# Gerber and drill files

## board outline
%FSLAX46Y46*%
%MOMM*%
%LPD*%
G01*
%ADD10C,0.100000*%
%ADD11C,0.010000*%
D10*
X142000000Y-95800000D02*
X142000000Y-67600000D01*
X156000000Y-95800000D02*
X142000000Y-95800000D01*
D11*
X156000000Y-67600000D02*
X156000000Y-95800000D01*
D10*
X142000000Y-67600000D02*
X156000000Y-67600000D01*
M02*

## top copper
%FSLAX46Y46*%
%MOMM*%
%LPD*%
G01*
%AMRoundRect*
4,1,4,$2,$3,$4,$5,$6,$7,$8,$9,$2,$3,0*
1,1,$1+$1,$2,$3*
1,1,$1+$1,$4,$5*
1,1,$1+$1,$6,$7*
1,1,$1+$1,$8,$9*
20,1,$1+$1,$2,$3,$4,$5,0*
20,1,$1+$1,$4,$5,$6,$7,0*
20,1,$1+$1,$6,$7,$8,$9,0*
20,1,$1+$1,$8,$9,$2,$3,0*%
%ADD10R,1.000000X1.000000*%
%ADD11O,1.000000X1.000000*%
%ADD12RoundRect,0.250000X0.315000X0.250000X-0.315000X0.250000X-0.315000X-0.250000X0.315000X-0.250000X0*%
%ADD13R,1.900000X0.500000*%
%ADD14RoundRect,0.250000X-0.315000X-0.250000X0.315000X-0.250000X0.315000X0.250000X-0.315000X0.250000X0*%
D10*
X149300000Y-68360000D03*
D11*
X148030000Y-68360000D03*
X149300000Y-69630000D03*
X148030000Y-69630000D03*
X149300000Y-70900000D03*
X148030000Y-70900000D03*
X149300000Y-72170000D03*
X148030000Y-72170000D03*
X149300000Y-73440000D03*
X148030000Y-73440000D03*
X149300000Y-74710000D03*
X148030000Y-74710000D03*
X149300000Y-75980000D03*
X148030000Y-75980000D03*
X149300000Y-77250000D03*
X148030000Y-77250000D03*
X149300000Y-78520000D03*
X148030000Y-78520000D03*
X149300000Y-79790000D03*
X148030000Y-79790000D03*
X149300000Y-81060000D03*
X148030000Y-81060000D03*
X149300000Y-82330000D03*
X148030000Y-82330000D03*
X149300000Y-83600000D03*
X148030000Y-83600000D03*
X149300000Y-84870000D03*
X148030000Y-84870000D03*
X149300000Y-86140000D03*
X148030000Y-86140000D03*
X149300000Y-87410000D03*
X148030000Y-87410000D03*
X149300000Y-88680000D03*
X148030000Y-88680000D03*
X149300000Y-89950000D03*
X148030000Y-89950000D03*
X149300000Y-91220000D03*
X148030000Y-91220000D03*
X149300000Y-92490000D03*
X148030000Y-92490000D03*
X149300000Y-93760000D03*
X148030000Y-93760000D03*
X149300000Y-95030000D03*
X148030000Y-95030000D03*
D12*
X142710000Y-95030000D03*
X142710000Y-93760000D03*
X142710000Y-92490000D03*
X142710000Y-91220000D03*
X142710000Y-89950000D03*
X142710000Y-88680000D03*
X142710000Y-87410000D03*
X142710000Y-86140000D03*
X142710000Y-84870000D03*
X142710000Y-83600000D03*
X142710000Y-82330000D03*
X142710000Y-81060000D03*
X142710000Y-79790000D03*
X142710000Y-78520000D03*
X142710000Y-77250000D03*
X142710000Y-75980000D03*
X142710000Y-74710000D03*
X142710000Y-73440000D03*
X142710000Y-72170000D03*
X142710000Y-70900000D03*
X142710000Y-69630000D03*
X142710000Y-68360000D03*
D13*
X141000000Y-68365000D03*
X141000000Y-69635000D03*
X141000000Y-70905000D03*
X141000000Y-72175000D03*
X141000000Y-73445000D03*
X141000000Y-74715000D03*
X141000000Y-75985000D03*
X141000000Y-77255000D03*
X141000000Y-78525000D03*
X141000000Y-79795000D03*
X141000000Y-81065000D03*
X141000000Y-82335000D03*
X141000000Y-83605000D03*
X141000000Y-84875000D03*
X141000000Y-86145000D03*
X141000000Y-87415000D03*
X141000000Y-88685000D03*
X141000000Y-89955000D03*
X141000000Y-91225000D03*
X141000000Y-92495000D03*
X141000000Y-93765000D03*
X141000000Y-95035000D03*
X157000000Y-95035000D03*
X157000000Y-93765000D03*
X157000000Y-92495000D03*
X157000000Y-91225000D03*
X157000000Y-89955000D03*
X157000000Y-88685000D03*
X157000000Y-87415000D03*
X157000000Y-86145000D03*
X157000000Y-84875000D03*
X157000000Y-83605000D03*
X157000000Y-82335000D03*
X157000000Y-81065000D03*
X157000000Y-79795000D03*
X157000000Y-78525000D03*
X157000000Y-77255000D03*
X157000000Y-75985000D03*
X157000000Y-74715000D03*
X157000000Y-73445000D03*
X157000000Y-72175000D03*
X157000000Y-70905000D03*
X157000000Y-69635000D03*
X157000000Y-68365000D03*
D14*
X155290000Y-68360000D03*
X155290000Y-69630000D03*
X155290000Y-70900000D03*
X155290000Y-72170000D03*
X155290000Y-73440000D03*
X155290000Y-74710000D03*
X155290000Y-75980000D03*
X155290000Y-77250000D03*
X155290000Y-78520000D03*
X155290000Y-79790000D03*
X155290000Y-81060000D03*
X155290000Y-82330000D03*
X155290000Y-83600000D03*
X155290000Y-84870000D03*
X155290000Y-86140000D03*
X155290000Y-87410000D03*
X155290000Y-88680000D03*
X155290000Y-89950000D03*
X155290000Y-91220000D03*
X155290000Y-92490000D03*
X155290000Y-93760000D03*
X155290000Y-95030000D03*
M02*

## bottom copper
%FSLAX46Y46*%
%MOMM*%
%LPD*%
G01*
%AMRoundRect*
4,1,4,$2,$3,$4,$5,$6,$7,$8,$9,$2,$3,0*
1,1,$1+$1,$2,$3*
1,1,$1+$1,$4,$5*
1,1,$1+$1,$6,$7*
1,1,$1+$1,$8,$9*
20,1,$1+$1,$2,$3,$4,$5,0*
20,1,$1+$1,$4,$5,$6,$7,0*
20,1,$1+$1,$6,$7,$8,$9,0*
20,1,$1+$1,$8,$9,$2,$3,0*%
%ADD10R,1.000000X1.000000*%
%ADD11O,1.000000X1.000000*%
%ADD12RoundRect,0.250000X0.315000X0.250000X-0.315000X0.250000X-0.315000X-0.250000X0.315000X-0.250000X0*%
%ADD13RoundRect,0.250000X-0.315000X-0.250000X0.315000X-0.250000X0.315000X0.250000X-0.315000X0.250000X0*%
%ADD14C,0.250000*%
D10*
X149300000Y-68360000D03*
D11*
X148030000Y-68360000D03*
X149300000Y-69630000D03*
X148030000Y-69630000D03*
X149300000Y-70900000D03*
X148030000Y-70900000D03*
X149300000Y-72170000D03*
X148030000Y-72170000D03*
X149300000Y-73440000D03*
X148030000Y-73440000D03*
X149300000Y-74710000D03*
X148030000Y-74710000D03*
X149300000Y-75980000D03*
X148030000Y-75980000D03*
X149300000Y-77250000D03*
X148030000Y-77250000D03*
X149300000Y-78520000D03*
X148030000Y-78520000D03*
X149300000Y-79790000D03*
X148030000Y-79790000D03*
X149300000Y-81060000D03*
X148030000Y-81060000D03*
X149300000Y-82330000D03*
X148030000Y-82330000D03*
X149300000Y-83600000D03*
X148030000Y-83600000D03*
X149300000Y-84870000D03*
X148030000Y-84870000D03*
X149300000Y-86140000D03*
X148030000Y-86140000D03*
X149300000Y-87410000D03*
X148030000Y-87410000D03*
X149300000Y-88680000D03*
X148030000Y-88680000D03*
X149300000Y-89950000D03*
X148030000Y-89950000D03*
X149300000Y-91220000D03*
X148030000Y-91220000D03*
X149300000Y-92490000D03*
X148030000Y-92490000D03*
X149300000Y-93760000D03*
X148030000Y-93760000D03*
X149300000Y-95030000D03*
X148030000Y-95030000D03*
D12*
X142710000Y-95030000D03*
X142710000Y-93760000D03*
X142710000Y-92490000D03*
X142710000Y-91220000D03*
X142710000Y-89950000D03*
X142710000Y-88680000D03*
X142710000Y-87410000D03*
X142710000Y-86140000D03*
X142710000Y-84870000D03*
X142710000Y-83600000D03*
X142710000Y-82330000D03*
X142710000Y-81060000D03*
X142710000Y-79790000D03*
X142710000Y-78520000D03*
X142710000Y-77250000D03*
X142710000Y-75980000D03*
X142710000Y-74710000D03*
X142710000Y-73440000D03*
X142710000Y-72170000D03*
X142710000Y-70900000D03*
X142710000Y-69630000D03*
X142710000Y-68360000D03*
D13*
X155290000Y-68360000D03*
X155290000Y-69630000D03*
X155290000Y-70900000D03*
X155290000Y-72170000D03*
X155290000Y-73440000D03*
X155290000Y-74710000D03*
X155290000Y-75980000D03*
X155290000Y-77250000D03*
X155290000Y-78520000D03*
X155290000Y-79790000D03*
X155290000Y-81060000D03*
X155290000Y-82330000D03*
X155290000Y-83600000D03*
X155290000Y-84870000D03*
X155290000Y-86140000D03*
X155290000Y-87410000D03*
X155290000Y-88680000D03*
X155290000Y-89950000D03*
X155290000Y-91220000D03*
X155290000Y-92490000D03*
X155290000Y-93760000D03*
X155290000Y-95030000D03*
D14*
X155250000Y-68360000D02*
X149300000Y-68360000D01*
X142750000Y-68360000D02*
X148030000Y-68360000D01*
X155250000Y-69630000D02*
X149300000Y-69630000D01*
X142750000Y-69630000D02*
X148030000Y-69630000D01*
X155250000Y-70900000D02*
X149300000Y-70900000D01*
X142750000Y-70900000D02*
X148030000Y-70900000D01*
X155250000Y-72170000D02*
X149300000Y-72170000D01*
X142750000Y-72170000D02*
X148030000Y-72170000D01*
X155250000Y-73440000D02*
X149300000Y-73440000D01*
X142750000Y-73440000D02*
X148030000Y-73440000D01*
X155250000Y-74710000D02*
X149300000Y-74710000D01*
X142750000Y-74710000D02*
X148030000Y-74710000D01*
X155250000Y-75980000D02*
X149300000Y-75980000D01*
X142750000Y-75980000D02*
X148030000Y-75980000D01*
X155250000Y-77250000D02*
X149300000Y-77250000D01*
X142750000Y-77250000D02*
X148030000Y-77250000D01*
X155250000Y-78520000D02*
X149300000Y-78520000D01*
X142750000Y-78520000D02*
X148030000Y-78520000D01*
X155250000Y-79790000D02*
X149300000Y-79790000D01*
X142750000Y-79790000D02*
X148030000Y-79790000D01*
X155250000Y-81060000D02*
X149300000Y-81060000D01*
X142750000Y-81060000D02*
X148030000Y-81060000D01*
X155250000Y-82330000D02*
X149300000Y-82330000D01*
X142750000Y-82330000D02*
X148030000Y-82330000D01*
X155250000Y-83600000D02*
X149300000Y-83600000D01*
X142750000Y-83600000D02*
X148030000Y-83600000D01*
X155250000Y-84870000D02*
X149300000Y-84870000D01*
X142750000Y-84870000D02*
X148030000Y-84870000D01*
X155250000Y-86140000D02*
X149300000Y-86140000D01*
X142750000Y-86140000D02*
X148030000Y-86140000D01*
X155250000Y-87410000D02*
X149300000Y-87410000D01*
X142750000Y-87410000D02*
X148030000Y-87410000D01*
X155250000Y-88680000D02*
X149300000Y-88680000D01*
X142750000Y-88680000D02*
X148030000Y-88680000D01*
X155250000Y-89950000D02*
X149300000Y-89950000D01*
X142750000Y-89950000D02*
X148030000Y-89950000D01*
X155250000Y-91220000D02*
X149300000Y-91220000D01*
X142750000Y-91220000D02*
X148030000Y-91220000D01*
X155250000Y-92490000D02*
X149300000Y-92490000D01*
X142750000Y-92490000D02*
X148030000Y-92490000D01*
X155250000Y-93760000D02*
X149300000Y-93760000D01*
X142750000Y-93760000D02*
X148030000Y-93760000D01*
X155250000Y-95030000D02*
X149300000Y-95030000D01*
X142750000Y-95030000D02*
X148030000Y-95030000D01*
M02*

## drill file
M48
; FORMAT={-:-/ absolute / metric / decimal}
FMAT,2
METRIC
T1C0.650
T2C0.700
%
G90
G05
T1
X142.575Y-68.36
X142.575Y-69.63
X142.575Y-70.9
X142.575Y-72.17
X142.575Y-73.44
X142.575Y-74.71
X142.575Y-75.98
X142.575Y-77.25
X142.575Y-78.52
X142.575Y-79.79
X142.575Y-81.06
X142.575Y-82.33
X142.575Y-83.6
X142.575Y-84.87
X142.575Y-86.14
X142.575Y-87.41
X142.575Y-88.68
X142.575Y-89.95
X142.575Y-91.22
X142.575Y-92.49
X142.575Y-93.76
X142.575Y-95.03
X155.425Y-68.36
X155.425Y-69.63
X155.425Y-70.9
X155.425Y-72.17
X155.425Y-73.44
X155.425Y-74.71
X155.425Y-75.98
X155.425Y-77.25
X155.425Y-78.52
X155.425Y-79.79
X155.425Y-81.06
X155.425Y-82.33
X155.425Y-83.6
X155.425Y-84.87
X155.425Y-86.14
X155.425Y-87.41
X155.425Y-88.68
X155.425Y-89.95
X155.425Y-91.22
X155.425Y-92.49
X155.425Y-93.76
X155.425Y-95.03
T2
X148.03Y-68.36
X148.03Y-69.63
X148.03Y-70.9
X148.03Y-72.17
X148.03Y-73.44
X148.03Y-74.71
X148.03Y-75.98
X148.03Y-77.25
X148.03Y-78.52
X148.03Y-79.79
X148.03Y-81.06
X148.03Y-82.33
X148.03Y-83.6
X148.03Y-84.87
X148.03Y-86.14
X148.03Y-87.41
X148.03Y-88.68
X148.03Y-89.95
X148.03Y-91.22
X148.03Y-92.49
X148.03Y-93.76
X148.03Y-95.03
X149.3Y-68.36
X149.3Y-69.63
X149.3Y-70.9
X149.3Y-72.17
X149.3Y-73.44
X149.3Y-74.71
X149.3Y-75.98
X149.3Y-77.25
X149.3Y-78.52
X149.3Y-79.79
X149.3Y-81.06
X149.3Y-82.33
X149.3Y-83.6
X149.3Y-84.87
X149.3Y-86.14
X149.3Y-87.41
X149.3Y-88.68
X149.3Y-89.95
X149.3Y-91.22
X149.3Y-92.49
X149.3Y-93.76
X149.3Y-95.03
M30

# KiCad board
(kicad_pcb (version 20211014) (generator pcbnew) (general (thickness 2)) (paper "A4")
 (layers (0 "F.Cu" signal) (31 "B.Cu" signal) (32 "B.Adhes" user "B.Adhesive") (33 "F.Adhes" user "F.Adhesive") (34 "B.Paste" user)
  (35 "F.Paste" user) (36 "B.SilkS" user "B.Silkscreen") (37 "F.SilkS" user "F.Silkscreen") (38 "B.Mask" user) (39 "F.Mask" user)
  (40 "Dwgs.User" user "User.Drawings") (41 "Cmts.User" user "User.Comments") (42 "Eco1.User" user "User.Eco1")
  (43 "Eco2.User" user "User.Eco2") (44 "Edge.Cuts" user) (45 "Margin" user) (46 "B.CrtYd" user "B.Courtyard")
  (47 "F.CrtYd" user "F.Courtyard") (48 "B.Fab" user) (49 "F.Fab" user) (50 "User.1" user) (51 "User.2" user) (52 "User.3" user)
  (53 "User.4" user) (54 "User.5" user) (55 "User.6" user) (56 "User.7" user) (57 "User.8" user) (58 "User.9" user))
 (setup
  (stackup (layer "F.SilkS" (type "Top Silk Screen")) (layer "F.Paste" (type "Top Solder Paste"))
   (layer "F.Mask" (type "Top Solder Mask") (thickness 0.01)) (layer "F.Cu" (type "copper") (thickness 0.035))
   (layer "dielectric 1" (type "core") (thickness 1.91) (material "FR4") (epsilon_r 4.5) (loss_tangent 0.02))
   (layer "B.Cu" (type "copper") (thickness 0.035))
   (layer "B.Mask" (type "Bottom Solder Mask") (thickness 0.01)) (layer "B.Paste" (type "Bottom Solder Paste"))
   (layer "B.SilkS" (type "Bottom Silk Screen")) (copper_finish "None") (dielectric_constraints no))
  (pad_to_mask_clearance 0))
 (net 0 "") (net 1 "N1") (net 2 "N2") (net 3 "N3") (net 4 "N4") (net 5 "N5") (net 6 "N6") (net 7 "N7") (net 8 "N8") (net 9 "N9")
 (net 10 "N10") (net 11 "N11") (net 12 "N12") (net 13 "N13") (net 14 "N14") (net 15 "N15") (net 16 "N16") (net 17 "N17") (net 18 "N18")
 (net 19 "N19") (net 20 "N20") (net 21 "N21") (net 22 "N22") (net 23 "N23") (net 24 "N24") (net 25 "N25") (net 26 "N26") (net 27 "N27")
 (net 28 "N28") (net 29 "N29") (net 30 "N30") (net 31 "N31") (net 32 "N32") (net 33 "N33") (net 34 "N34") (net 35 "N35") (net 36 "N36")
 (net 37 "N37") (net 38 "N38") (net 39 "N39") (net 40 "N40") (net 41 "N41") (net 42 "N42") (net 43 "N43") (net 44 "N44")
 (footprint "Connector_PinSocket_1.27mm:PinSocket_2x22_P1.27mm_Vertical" (layer "F.Cu") (at 149.3 68.36)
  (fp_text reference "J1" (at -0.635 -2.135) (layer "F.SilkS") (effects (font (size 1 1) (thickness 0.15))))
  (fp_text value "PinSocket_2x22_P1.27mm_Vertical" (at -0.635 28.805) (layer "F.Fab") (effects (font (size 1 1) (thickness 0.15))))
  (pad "1" thru_hole rect (at 0 0) (size 1 1) (drill 0.7) (layers *.Cu *.Mask) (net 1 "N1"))
  (pad "2" thru_hole oval (at -1.27 0) (size 1 1) (drill 0.7) (layers *.Cu *.Mask) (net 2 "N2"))
  (pad "3" thru_hole oval (at 0 1.27) (size 1 1) (drill 0.7) (layers *.Cu *.Mask) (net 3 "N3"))
  (pad "4" thru_hole oval (at -1.27 1.27) (size 1 1) (drill 0.7) (layers *.Cu *.Mask) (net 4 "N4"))
  (pad "5" thru_hole oval (at 0 2.54) (size 1 1) (drill 0.7) (layers *.Cu *.Mask) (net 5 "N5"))
  (pad "6" thru_hole oval (at -1.27 2.54) (size 1 1) (drill 0.7) (layers *.Cu *.Mask) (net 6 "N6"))
  (pad "7" thru_hole oval (at 0 3.81) (size 1 1) (drill 0.7) (layers *.Cu *.Mask) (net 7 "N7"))
  (pad "8" thru_hole oval (at -1.27 3.81) (size 1 1) (drill 0.7) (layers *.Cu *.Mask) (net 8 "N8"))
  (pad "9" thru_hole oval (at 0 5.08) (size 1 1) (drill 0.7) (layers *.Cu *.Mask) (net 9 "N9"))
  (pad "10" thru_hole oval (at -1.27 5.08) (size 1 1) (drill 0.7) (layers *.Cu *.Mask) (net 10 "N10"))
  (pad "11" thru_hole oval (at 0 6.35) (size 1 1) (drill 0.7) (layers *.Cu *.Mask) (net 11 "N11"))
  (pad "12" thru_hole oval (at -1.27 6.35) (size 1 1) (drill 0.7) (layers *.Cu *.Mask) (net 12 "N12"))
  (pad "13" thru_hole oval (at 0 7.62) (size 1 1) (drill 0.7) (layers *.Cu *.Mask) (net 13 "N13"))
  (pad "14" thru_hole oval (at -1.27 7.62) (size 1 1) (drill 0.7) (layers *.Cu *.Mask) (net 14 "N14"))
  (pad "15" thru_hole oval (at 0 8.89) (size 1 1) (drill 0.7) (layers *.Cu *.Mask) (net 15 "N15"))
  (pad "16" thru_hole oval (at -1.27 8.89) (size 1 1) (drill 0.7) (layers *.Cu *.Mask) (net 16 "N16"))
  (pad "17" thru_hole oval (at 0 10.16) (size 1 1) (drill 0.7) (layers *.Cu *.Mask) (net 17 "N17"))
  (pad "18" thru_hole oval (at -1.27 10.16) (size 1 1) (drill 0.7) (layers *.Cu *.Mask) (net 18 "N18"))
  (pad "19" thru_hole oval (at 0 11.43) (size 1 1) (drill 0.7) (layers *.Cu *.Mask) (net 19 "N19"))
  (pad "20" thru_hole oval (at -1.27 11.43) (size 1 1) (drill 0.7) (layers *.Cu *.Mask) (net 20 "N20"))
  (pad "21" thru_hole oval (at 0 12.7) (size 1 1) (drill 0.7) (layers *.Cu *.Mask) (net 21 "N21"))
  (pad "22" thru_hole oval (at -1.27 12.7) (size 1 1) (drill 0.7) (layers *.Cu *.Mask) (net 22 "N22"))
  (pad "23" thru_hole oval (at 0 13.97) (size 1 1) (drill 0.7) (layers *.Cu *.Mask) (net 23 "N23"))
  (pad "24" thru_hole oval (at -1.27 13.97) (size 1 1) (drill 0.7) (layers *.Cu *.Mask) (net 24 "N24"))
  (pad "25" thru_hole oval (at 0 15.24) (size 1 1) (drill 0.7) (layers *.Cu *.Mask) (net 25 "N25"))
  (pad "26" thru_hole oval (at -1.27 15.24) (size 1 1) (drill 0.7) (layers *.Cu *.Mask) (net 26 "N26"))
  (pad "27" thru_hole oval (at 0 16.51) (size 1 1) (drill 0.7) (layers *.Cu *.Mask) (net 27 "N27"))
  (pad "28" thru_hole oval (at -1.27 16.51) (size 1 1) (drill 0.7) (layers *.Cu *.Mask) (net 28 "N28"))
  (pad "29" thru_hole oval (at 0 17.78) (size 1 1) (drill 0.7) (layers *.Cu *.Mask) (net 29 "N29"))
  (pad "30" thru_hole oval (at -1.27 17.78) (size 1 1) (drill 0.7) (layers *.Cu *.Mask) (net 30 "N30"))
  (pad "31" thru_hole oval (at 0 19.05) (size 1 1) (drill 0.7) (layers *.Cu *.Mask) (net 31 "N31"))
  (pad "32" thru_hole oval (at -1.27 19.05) (size 1 1) (drill 0.7) (layers *.Cu *.Mask) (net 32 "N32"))
  (pad "33" thru_hole oval (at 0 20.32) (size 1 1) (drill 0.7) (layers *.Cu *.Mask) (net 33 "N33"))
  (pad "34" thru_hole oval (at -1.27 20.32) (size 1 1) (drill 0.7) (layers *.Cu *.Mask) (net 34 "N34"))
  (pad "35" thru_hole oval (at 0 21.59) (size 1 1) (drill 0.7) (layers *.Cu *.Mask) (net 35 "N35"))
  (pad "36" thru_hole oval (at -1.27 21.59) (size 1 1) (drill 0.7) (layers *.Cu *.Mask) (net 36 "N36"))
  (pad "37" thru_hole oval (at 0 22.86) (size 1 1) (drill 0.7) (layers *.Cu *.Mask) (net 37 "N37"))
  (pad "38" thru_hole oval (at -1.27 22.86) (size 1 1) (drill 0.7) (layers *.Cu *.Mask) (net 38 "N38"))
  (pad "39" thru_hole oval (at 0 24.13) (size 1 1) (drill 0.7) (layers *.Cu *.Mask) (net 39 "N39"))
  (pad "40" thru_hole oval (at -1.27 24.13) (size 1 1) (drill 0.7) (layers *.Cu *.Mask) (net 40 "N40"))
  (pad "41" thru_hole oval (at 0 25.4) (size 1 1) (drill 0.7) (layers *.Cu *.Mask) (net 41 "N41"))
  (pad "42" thru_hole oval (at -1.27 25.4) (size 1 1) (drill 0.7) (layers *.Cu *.Mask) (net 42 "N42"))
  (pad "43" thru_hole oval (at 0 26.67) (size 1 1) (drill 0.7) (layers *.Cu *.Mask) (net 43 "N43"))
  (pad "44" thru_hole oval (at -1.27 26.67) (size 1 1) (drill 0.7) (layers *.Cu *.Mask) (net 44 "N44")))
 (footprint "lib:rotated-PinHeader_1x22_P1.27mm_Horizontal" (layer "F.Cu") (at 142.575 95.03 180)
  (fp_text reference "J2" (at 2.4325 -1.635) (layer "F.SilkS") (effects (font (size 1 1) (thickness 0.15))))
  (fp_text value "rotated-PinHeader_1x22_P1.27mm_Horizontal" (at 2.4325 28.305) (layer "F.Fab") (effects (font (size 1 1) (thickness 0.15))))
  (pad "1" thru_hole roundrect (at 0 0 180) (size 1.13 1) (drill 0.65 (offset -0.135 0)) (layers *.Cu *.Mask) (roundrect_rratio 0.25)
   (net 44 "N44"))
  (pad "2" thru_hole roundrect (at 0 1.27 180) (size 1.13 1) (drill 0.65 (offset -0.135 0)) (layers *.Cu *.Mask) (roundrect_rratio 0.25)
   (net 42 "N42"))
  (pad "3" thru_hole roundrect (at 0 2.54 180) (size 1.13 1) (drill 0.65 (offset -0.135 0)) (layers *.Cu *.Mask) (roundrect_rratio 0.25)
   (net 40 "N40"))
  (pad "4" thru_hole roundrect (at 0 3.81 180) (size 1.13 1) (drill 0.65 (offset -0.135 0)) (layers *.Cu *.Mask) (roundrect_rratio 0.25)
   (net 38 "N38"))
  (pad "5" thru_hole roundrect (at 0 5.08 180) (size 1.13 1) (drill 0.65 (offset -0.135 0)) (layers *.Cu *.Mask) (roundrect_rratio 0.25)
   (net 36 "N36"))
  (pad "6" thru_hole roundrect (at 0 6.35 180) (size 1.13 1) (drill 0.65 (offset -0.135 0)) (layers *.Cu *.Mask) (roundrect_rratio 0.25)
   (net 34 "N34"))
  (pad "7" thru_hole roundrect (at 0 7.62 180) (size 1.13 1) (drill 0.65 (offset -0.135 0)) (layers *.Cu *.Mask) (roundrect_rratio 0.25)
   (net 32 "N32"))
  (pad "8" thru_hole roundrect (at 0 8.89 180) (size 1.13 1) (drill 0.65 (offset -0.135 0)) (layers *.Cu *.Mask) (roundrect_rratio 0.25)
   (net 30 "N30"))
  (pad "9" thru_hole roundrect (at 0 10.16 180) (size 1.13 1) (drill 0.65 (offset -0.135 0)) (layers *.Cu *.Mask) (roundrect_rratio 0.25)
   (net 28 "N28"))
  (pad "10" thru_hole roundrect (at 0 11.43 180) (size 1.13 1) (drill 0.65 (offset -0.135 0)) (layers *.Cu *.Mask) (roundrect_rratio 0.25)
   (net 26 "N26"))
  (pad "11" thru_hole roundrect (at 0 12.7 180) (size 1.13 1) (drill 0.65 (offset -0.135 0)) (layers *.Cu *.Mask) (roundrect_rratio 0.25)
   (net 24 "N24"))
  (pad "12" thru_hole roundrect (at 0 13.97 180) (size 1.13 1) (drill 0.65 (offset -0.135 0)) (layers *.Cu *.Mask) (roundrect_rratio 0.25)
   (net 22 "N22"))
  (pad "13" thru_hole roundrect (at 0 15.24 180) (size 1.13 1) (drill 0.65 (offset -0.135 0)) (layers *.Cu *.Mask) (roundrect_rratio 0.25)
   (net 20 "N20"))
  (pad "14" thru_hole roundrect (at 0 16.51 180) (size 1.13 1) (drill 0.65 (offset -0.135 0)) (layers *.Cu *.Mask) (roundrect_rratio 0.25)
   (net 18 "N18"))
  (pad "15" thru_hole roundrect (at 0 17.78 180) (size 1.13 1) (drill 0.65 (offset -0.135 0)) (layers *.Cu *.Mask) (roundrect_rratio 0.25)
   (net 16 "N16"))
  (pad "16" thru_hole roundrect (at 0 19.05 180) (size 1.13 1) (drill 0.65 (offset -0.135 0)) (layers *.Cu *.Mask) (roundrect_rratio 0.25)
   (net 14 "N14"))
  (pad "17" thru_hole roundrect (at 0 20.32 180) (size 1.13 1) (drill 0.65 (offset -0.135 0)) (layers *.Cu *.Mask) (roundrect_rratio 0.25)
   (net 12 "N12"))
  (pad "18" thru_hole roundrect (at 0 21.59 180) (size 1.13 1) (drill 0.65 (offset -0.135 0)) (layers *.Cu *.Mask) (roundrect_rratio 0.25)
   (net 10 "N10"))
  (pad "19" thru_hole roundrect (at 0 22.86 180) (size 1.13 1) (drill 0.65 (offset -0.135 0)) (layers *.Cu *.Mask) (roundrect_rratio 0.25)
   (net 8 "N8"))
  (pad "20" thru_hole roundrect (at 0 24.13 180) (size 1.13 1) (drill 0.65 (offset -0.135 0)) (layers *.Cu *.Mask) (roundrect_rratio 0.25)
   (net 6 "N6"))
  (pad "21" thru_hole roundrect (at 0 25.4 180) (size 1.13 1) (drill 0.65 (offset -0.135 0)) (layers *.Cu *.Mask) (roundrect_rratio 0.25)
   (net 4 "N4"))
  (pad "22" thru_hole roundrect (at 0 26.67 180) (size 1.13 1) (drill 0.65 (offset -0.135 0)) (layers *.Cu *.Mask) (roundrect_rratio 0.25)
   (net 2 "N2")))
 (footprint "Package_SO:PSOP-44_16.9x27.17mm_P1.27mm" (layer "F.Cu") (at 149 81.7)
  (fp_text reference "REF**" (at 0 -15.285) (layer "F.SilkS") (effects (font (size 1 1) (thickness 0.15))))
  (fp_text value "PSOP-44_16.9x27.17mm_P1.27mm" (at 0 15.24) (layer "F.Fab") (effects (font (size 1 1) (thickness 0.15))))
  (pad "1" smd rect (at -8 -13.335 270) (size 0.5 1.9) (layers "F.Cu" "F.Paste" "F.Mask"))
  (pad "2" smd rect (at -8 -12.065 270) (size 0.5 1.9) (layers "F.Cu" "F.Paste" "F.Mask"))
  (pad "3" smd rect (at -8 -10.795 270) (size 0.5 1.9) (layers "F.Cu" "F.Paste" "F.Mask"))
  (pad "4" smd rect (at -8 -9.525 270) (size 0.5 1.9) (layers "F.Cu" "F.Paste" "F.Mask"))
  (pad "5" smd rect (at -8 -8.255 270) (size 0.5 1.9) (layers "F.Cu" "F.Paste" "F.Mask"))
  (pad "6" smd rect (at -8 -6.985 270) (size 0.5 1.9) (layers "F.Cu" "F.Paste" "F.Mask"))
  (pad "7" smd rect (at -8 -5.715 270) (size 0.5 1.9) (layers "F.Cu" "F.Paste" "F.Mask"))
  (pad "8" smd rect (at -8 -4.445 270) (size 0.5 1.9) (layers "F.Cu" "F.Paste" "F.Mask"))
  (pad "9" smd rect (at -8 -3.175 270) (size 0.5 1.9) (layers "F.Cu" "F.Paste" "F.Mask"))
  (pad "10" smd rect (at -8 -1.905 270) (size 0.5 1.9) (layers "F.Cu" "F.Paste" "F.Mask"))
  (pad "11" smd rect (at -8 -0.635 270) (size 0.5 1.9) (layers "F.Cu" "F.Paste" "F.Mask"))
  (pad "12" smd rect (at -8 0.635 270) (size 0.5 1.9) (layers "F.Cu" "F.Paste" "F.Mask"))
  (pad "13" smd rect (at -8 1.905 270) (size 0.5 1.9) (layers "F.Cu" "F.Paste" "F.Mask"))
  (pad "14" smd rect (at -8 3.175 270) (size 0.5 1.9) (layers "F.Cu" "F.Paste" "F.Mask"))
  (pad "15" smd rect (at -8 4.445 270) (size 0.5 1.9) (layers "F.Cu" "F.Paste" "F.Mask"))
  (pad "16" smd rect (at -8 5.715 270) (size 0.5 1.9) (layers "F.Cu" "F.Paste" "F.Mask"))
  (pad "17" smd rect (at -8 6.985 270) (size 0.5 1.9) (layers "F.Cu" "F.Paste" "F.Mask"))
  (pad "18" smd rect (at -8 8.255 270) (size 0.5 1.9) (layers "F.Cu" "F.Paste" "F.Mask"))
  (pad "19" smd rect (at -8 9.525 270) (size 0.5 1.9) (layers "F.Cu" "F.Paste" "F.Mask"))
  (pad "20" smd rect (at -8 10.795 270) (size 0.5 1.9) (layers "F.Cu" "F.Paste" "F.Mask"))
  (pad "21" smd rect (at -8 12.065 270) (size 0.5 1.9) (layers "F.Cu" "F.Paste" "F.Mask"))
  (pad "22" smd rect (at -8 13.335 270) (size 0.5 1.9) (layers "F.Cu" "F.Paste" "F.Mask"))
  (pad "23" smd rect (at 8 13.335 270) (size 0.5 1.9) (layers "F.Cu" "F.Paste" "F.Mask"))
  (pad "24" smd rect (at 8 12.065 270) (size 0.5 1.9) (layers "F.Cu" "F.Paste" "F.Mask"))
  (pad "25" smd rect (at 8 10.795 270) (size 0.5 1.9) (layers "F.Cu" "F.Paste" "F.Mask"))
  (pad "26" smd rect (at 8 9.525 270) (size 0.5 1.9) (layers "F.Cu" "F.Paste" "F.Mask"))
  (pad "27" smd rect (at 8 8.255 270) (size 0.5 1.9) (layers "F.Cu" "F.Paste" "F.Mask"))
  (pad "28" smd rect (at 8 6.985 270) (size 0.5 1.9) (layers "F.Cu" "F.Paste" "F.Mask"))
  (pad "29" smd rect (at 8 5.715 270) (size 0.5 1.9) (layers "F.Cu" "F.Paste" "F.Mask"))
  (pad "30" smd rect (at 8 4.445 270) (size 0.5 1.9) (layers "F.Cu" "F.Paste" "F.Mask"))
  (pad "31" smd rect (at 8 3.175 270) (size 0.5 1.9) (layers "F.Cu" "F.Paste" "F.Mask"))
  (pad "32" smd rect (at 8 1.905 270) (size 0.5 1.9) (layers "F.Cu" "F.Paste" "F.Mask"))
  (pad "33" smd rect (at 8 0.635 270) (size 0.5 1.9) (layers "F.Cu" "F.Paste" "F.Mask"))
  (pad "34" smd rect (at 8 -0.635 270) (size 0.5 1.9) (layers "F.Cu" "F.Paste" "F.Mask"))
  (pad "35" smd rect (at 8 -1.905 270) (size 0.5 1.9) (layers "F.Cu" "F.Paste" "F.Mask"))
  (pad "36" smd rect (at 8 -3.175 270) (size 0.5 1.9) (layers "F.Cu" "F.Paste" "F.Mask"))
  (pad "37" smd rect (at 8 -4.445 270) (size 0.5 1.9) (layers "F.Cu" "F.Paste" "F.Mask"))
  (pad "38" smd rect (at 8 -5.715 270) (size 0.5 1.9) (layers "F.Cu" "F.Paste" "F.Mask"))
  (pad "39" smd rect (at 8 -6.985 270) (size 0.5 1.9) (layers "F.Cu" "F.Paste" "F.Mask"))
  (pad "40" smd rect (at 8 -8.255 270) (size 0.5 1.9) (layers "F.Cu" "F.Paste" "F.Mask"))
  (pad "41" smd rect (at 8 -9.525 270) (size 0.5 1.9) (layers "F.Cu" "F.Paste" "F.Mask"))
  (pad "42" smd rect (at 8 -10.795 270) (size 0.5 1.9) (layers "F.Cu" "F.Paste" "F.Mask"))
  (pad "43" smd rect (at 8 -12.065 270) (size 0.5 1.9) (layers "F.Cu" "F.Paste" "F.Mask"))
  (pad "44" smd rect (at 8 -13.335 270) (size 0.5 1.9) (layers "F.Cu" "F.Paste" "F.Mask")))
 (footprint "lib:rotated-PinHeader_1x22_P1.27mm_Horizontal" (layer "F.Cu") (at 155.425 68.36)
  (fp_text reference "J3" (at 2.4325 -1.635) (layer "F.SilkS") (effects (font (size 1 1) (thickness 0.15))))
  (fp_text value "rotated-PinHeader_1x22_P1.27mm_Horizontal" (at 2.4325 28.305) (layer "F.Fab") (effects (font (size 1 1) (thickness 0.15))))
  (pad "1" thru_hole roundrect (at 0 0) (size 1.13 1) (drill 0.65 (offset -0.135 0)) (layers *.Cu *.Mask) (roundrect_rratio 0.25)
   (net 1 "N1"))
  (pad "2" thru_hole roundrect (at 0 1.27) (size 1.13 1) (drill 0.65 (offset -0.135 0)) (layers *.Cu *.Mask) (roundrect_rratio 0.25)
   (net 3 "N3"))
  (pad "3" thru_hole roundrect (at 0 2.54) (size 1.13 1) (drill 0.65 (offset -0.135 0)) (layers *.Cu *.Mask) (roundrect_rratio 0.25)
   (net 5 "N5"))
  (pad "4" thru_hole roundrect (at 0 3.81) (size 1.13 1) (drill 0.65 (offset -0.135 0)) (layers *.Cu *.Mask) (roundrect_rratio 0.25)
   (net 7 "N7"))
  (pad "5" thru_hole roundrect (at 0 5.08) (size 1.13 1) (drill 0.65 (offset -0.135 0)) (layers *.Cu *.Mask) (roundrect_rratio 0.25)
   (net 9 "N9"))
  (pad "6" thru_hole roundrect (at 0 6.35) (size 1.13 1) (drill 0.65 (offset -0.135 0)) (layers *.Cu *.Mask) (roundrect_rratio 0.25)
   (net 11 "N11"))
  (pad "7" thru_hole roundrect (at 0 7.62) (size 1.13 1) (drill 0.65 (offset -0.135 0)) (layers *.Cu *.Mask) (roundrect_rratio 0.25)
   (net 13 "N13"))
  (pad "8" thru_hole roundrect (at 0 8.89) (size 1.13 1) (drill 0.65 (offset -0.135 0)) (layers *.Cu *.Mask) (roundrect_rratio 0.25)
   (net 15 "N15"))
  (pad "9" thru_hole roundrect (at 0 10.16) (size 1.13 1) (drill 0.65 (offset -0.135 0)) (layers *.Cu *.Mask) (roundrect_rratio 0.25)
   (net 17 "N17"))
  (pad "10" thru_hole roundrect (at 0 11.43) (size 1.13 1) (drill 0.65 (offset -0.135 0)) (layers *.Cu *.Mask) (roundrect_rratio 0.25)
   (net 19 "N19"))
  (pad "11" thru_hole roundrect (at 0 12.7) (size 1.13 1) (drill 0.65 (offset -0.135 0)) (layers *.Cu *.Mask) (roundrect_rratio 0.25)
   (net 21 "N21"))
  (pad "12" thru_hole roundrect (at 0 13.97) (size 1.13 1) (drill 0.65 (offset -0.135 0)) (layers *.Cu *.Mask) (roundrect_rratio 0.25)
   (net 23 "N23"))
  (pad "13" thru_hole roundrect (at 0 15.24) (size 1.13 1) (drill 0.65 (offset -0.135 0)) (layers *.Cu *.Mask) (roundrect_rratio 0.25)
   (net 25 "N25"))
  (pad "14" thru_hole roundrect (at 0 16.51) (size 1.13 1) (drill 0.65 (offset -0.135 0)) (layers *.Cu *.Mask) (roundrect_rratio 0.25)
   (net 27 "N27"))
  (pad "15" thru_hole roundrect (at 0 17.78) (size 1.13 1) (drill 0.65 (offset -0.135 0)) (layers *.Cu *.Mask) (roundrect_rratio 0.25)
   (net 29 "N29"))
  (pad "16" thru_hole roundrect (at 0 19.05) (size 1.13 1) (drill 0.65 (offset -0.135 0)) (layers *.Cu *.Mask) (roundrect_rratio 0.25)
   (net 31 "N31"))
  (pad "17" thru_hole roundrect (at 0 20.32) (size 1.13 1) (drill 0.65 (offset -0.135 0)) (layers *.Cu *.Mask) (roundrect_rratio 0.25)
   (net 33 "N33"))
  (pad "18" thru_hole roundrect (at 0 21.59) (size 1.13 1) (drill 0.65 (offset -0.135 0)) (layers *.Cu *.Mask) (roundrect_rratio 0.25)
   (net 35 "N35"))
  (pad "19" thru_hole roundrect (at 0 22.86) (size 1.13 1) (drill 0.65 (offset -0.135 0)) (layers *.Cu *.Mask) (roundrect_rratio 0.25)
   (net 37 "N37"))
  (pad "20" thru_hole roundrect (at 0 24.13) (size 1.13 1) (drill 0.65 (offset -0.135 0)) (layers *.Cu *.Mask) (roundrect_rratio 0.25)
   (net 39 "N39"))
  (pad "21" thru_hole roundrect (at 0 25.4) (size 1.13 1) (drill 0.65 (offset -0.135 0)) (layers *.Cu *.Mask) (roundrect_rratio 0.25)
   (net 41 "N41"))
  (pad "22" thru_hole roundrect (at 0 26.67) (size 1.13 1) (drill 0.65 (offset -0.135 0)) (layers *.Cu *.Mask) (roundrect_rratio 0.25)
   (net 43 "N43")))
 (gr_line (start 142 95.8) (end 142 67.6) (layer "Edge.Cuts") (width 0.1))
 (gr_line (start 156 95.8) (end 142 95.8) (layer "Edge.Cuts") (width 0.1))
 (gr_line (start 156 67.6) (end 156 95.8) (layer "Edge.Cuts") (width 0.01))
 (gr_line (start 142 67.6) (end 156 67.6) (layer "Edge.Cuts") (width 0.1))
 (segment (start 155.25 68.36) (end 149.3 68.36) (width 0.25) (layer "B.Cu") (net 1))
 (segment (start 142.75 68.36) (end 148.03 68.36) (width 0.25) (layer "B.Cu") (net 2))
 (segment (start 155.25 69.63) (end 149.3 69.63) (width 0.25) (layer "B.Cu") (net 3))
 (segment (start 142.75 69.63) (end 148.03 69.63) (width 0.25) (layer "B.Cu") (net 4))
 (segment (start 155.25 70.9) (end 149.3 70.9) (width 0.25) (layer "B.Cu") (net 5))
 (segment (start 142.75 70.9) (end 148.03 70.9) (width 0.25) (layer "B.Cu") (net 6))
 (segment (start 155.25 72.17) (end 149.3 72.17) (width 0.25) (layer "B.Cu") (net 7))
 (segment (start 142.75 72.17) (end 148.03 72.17) (width 0.25) (layer "B.Cu") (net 8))
 (segment (start 155.25 73.44) (end 149.3 73.44) (width 0.25) (layer "B.Cu") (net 9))
 (segment (start 142.75 73.44) (end 148.03 73.44) (width 0.25) (layer "B.Cu") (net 10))
 (segment (start 155.25 74.71) (end 149.3 74.71) (width 0.25) (layer "B.Cu") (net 11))
 (segment (start 142.75 74.71) (end 148.03 74.71) (width 0.25) (layer "B.Cu") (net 12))
 (segment (start 155.25 75.98) (end 149.3 75.98) (width 0.25) (layer "B.Cu") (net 13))
 (segment (start 142.75 75.98) (end 148.03 75.98) (width 0.25) (layer "B.Cu") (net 14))
 (segment (start 155.25 77.25) (end 149.3 77.25) (width 0.25) (layer "B.Cu") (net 15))
 (segment (start 142.75 77.25) (end 148.03 77.25) (width 0.25) (layer "B.Cu") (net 16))
 (segment (start 155.25 78.52) (end 149.3 78.52) (width 0.25) (layer "B.Cu") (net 17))
 (segment (start 142.75 78.52) (end 148.03 78.52) (width 0.25) (layer "B.Cu") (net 18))
 (segment (start 155.25 79.79) (end 149.3 79.79) (width 0.25) (layer "B.Cu") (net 19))
 (segment (start 142.75 79.79) (end 148.03 79.79) (width 0.25) (layer "B.Cu") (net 20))
 (segment (start 155.25 81.06) (end 149.3 81.06) (width 0.25) (layer "B.Cu") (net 21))
 (segment (start 142.75 81.06) (end 148.03 81.06) (width 0.25) (layer "B.Cu") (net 22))
 (segment (start 155.25 82.33) (end 149.3 82.33) (width 0.25) (layer "B.Cu") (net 23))
 (segment (start 142.75 82.33) (end 148.03 82.33) (width 0.25) (layer "B.Cu") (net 24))
 (segment (start 155.25 83.6) (end 149.3 83.6) (width 0.25) (layer "B.Cu") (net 25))
 (segment (start 142.75 83.6) (end 148.03 83.6) (width 0.25) (layer "B.Cu") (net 26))
 (segment (start 155.25 84.87) (end 149.3 84.87) (width 0.25) (layer "B.Cu") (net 27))
 (segment (start 142.75 84.87) (end 148.03 84.87) (width 0.25) (layer "B.Cu") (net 28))
 (segment (start 155.25 86.14) (end 149.3 86.14) (width 0.25) (layer "B.Cu") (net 29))
 (segment (start 142.75 86.14) (end 148.03 86.14) (width 0.25) (layer "B.Cu") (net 30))
 (segment (start 155.25 87.41) (end 149.3 87.41) (width 0.25) (layer "B.Cu") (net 31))
 (segment (start 142.75 87.41) (end 148.03 87.41) (width 0.25) (layer "B.Cu") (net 32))
 (segment (start 155.25 88.68) (end 149.3 88.68) (width 0.25) (layer "B.Cu") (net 33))
 (segment (start 142.75 88.68) (end 148.03 88.68) (width 0.25) (layer "B.Cu") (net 34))
 (segment (start 155.25 89.95) (end 149.3 89.95) (width 0.25) (layer "B.Cu") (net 35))
 (segment (start 142.75 89.95) (end 148.03 89.95) (width 0.25) (layer "B.Cu") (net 36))
 (segment (start 155.25 91.22) (end 149.3 91.22) (width 0.25) (layer "B.Cu") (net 37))
 (segment (start 142.75 91.22) (end 148.03 91.22) (width 0.25) (layer "B.Cu") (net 38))
 (segment (start 155.25 92.49) (end 149.3 92.49) (width 0.25) (layer "B.Cu") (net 39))
 (segment (start 142.75 92.49) (end 148.03 92.49) (width 0.25) (layer "B.Cu") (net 40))
 (segment (start 155.25 93.76) (end 149.3 93.76) (width 0.25) (layer "B.Cu") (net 41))
 (segment (start 142.75 93.76) (end 148.03 93.76) (width 0.25) (layer "B.Cu") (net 42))
 (segment (start 155.25 95.03) (end 149.3 95.03) (width 0.25) (layer "B.Cu") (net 43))
 (segment (start 142.75 95.03) (end 148.03 95.03) (width 0.25) (layer "B.Cu") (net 44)))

